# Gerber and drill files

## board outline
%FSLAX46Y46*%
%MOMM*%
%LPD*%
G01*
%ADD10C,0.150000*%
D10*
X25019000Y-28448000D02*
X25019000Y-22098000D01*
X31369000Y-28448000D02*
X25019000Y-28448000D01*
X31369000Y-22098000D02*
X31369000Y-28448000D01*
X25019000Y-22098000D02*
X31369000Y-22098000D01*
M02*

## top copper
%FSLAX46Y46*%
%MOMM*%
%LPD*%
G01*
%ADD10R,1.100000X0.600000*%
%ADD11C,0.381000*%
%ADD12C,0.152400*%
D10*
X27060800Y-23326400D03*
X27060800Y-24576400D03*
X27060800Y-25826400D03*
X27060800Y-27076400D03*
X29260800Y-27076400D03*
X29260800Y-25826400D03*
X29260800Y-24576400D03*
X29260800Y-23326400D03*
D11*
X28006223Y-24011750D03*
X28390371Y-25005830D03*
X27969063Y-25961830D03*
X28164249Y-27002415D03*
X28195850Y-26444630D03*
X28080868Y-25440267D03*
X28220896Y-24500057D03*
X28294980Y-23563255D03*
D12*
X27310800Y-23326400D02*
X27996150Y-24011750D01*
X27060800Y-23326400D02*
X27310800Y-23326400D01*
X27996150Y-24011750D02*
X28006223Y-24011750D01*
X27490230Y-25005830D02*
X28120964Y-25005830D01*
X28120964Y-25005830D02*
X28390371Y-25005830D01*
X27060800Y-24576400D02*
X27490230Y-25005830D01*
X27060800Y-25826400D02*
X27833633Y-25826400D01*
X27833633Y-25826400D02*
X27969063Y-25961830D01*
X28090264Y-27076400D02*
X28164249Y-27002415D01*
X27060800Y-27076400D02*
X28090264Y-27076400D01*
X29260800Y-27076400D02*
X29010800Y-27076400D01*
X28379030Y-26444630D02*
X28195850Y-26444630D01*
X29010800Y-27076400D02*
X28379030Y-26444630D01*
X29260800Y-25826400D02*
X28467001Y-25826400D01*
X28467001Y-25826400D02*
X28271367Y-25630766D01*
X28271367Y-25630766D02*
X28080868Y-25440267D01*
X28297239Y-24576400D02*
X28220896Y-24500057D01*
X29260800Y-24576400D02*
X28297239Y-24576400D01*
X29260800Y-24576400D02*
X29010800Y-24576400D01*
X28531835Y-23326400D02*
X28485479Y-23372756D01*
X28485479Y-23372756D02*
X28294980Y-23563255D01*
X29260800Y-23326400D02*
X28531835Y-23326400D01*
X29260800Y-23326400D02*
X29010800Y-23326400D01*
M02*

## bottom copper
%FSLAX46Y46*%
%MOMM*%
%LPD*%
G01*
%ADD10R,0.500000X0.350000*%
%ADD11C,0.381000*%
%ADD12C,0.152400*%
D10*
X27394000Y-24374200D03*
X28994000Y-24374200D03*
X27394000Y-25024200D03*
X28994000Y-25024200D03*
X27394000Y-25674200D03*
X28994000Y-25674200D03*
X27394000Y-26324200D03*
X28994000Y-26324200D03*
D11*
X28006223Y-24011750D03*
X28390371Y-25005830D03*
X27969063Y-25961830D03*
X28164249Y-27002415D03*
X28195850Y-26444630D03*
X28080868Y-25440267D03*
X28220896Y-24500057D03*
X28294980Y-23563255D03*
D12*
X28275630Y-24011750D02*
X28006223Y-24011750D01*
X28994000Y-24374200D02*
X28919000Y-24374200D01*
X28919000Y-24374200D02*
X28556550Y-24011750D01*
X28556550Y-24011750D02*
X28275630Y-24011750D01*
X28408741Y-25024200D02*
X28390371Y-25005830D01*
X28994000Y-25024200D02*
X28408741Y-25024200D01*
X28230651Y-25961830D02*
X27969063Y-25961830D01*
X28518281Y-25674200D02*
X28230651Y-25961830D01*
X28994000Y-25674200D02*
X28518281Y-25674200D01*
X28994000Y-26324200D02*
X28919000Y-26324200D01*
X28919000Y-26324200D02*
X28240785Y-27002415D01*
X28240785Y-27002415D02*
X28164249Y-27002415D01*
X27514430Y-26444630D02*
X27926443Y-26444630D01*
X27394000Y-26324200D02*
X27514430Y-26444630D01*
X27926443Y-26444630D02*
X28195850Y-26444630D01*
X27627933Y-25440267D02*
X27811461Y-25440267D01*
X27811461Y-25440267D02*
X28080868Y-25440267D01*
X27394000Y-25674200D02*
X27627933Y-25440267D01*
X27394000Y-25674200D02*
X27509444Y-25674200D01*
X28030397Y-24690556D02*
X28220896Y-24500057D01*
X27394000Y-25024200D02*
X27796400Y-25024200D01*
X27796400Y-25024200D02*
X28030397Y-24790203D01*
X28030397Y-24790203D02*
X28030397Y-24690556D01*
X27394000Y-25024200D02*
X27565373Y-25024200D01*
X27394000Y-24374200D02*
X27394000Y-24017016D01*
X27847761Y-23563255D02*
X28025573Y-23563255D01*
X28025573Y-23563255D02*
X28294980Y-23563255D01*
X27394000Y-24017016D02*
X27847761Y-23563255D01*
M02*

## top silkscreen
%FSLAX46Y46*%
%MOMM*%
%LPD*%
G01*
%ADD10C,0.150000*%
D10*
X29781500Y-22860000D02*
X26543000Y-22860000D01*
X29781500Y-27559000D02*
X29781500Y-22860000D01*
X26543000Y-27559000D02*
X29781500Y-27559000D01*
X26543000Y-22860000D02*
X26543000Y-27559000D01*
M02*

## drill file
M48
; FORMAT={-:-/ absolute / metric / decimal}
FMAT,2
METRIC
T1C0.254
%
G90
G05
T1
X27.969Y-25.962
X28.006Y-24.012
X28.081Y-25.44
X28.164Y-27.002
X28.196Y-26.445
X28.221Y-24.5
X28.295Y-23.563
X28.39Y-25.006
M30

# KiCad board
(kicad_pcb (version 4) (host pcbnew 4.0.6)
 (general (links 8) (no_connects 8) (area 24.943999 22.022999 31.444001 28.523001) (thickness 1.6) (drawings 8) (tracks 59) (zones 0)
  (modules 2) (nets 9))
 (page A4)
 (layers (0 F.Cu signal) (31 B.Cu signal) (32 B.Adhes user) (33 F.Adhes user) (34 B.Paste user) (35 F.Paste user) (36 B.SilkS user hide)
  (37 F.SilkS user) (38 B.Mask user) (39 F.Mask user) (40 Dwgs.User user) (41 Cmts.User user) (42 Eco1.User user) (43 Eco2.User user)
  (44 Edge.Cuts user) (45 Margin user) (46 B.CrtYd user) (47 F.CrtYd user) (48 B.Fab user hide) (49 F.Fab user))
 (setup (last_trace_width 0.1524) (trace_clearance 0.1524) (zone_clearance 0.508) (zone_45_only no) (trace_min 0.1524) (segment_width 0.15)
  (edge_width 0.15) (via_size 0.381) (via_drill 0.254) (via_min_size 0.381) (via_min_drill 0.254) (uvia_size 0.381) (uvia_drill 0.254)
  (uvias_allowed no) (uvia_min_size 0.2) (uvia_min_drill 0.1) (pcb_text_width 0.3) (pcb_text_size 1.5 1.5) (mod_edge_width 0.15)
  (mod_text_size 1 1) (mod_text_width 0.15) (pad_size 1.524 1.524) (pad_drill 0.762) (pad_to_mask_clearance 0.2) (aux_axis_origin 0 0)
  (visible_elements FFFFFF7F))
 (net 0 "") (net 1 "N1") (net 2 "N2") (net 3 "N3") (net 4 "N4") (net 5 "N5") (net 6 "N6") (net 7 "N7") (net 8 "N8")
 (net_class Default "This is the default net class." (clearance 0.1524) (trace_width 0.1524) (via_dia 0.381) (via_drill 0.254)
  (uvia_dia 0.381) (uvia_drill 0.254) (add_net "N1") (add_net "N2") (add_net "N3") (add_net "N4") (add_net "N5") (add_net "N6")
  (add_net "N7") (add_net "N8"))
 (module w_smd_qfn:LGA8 (layer F.Cu) (at 28.1608 25.2264)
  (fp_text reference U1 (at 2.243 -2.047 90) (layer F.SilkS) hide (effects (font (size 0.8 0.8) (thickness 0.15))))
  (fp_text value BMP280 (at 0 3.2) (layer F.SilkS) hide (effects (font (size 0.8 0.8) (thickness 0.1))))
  (pad 1 smd rect (at -1.1 -1.9) (size 1.1 0.6) (layers F.Cu F.Paste F.Mask) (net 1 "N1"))
  (pad 2 smd rect (at -1.1 -0.65) (size 1.1 0.6) (layers F.Cu F.Paste F.Mask) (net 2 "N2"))
  (pad 3 smd rect (at -1.1 0.6) (size 1.1 0.6) (layers F.Cu F.Paste F.Mask) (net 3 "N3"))
  (pad 4 smd rect (at -1.1 1.85) (size 1.1 0.6) (layers F.Cu F.Paste F.Mask) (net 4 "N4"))
  (pad 5 smd rect (at 1.1 1.85) (size 1.1 0.6) (layers F.Cu F.Paste F.Mask) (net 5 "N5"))
  (pad 6 smd rect (at 1.1 0.6) (size 1.1 0.6) (layers F.Cu F.Paste F.Mask) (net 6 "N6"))
  (pad 7 smd rect (at 1.1 -0.65) (size 1.1 0.6) (layers F.Cu F.Paste F.Mask) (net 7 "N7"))
  (pad 8 smd rect (at 1.1 -1.9) (size 1.1 0.6) (layers F.Cu F.Paste F.Mask) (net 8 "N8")))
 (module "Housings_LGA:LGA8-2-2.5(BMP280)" (layer B.Cu) (at 28.194 25.3492 270)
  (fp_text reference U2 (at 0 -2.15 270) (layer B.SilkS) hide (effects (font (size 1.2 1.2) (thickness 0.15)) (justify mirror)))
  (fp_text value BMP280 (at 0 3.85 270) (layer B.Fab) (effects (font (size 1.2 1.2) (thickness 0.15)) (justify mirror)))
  (pad 1 smd rect (at -0.975 0.8 270) (size 0.35 0.5) (layers B.Cu B.Paste B.Mask) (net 8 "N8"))
  (pad 8 smd rect (at -0.975 -0.8 270) (size 0.35 0.5) (layers B.Cu B.Paste B.Mask) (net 1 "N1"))
  (pad 2 smd rect (at -0.325 0.8 270) (size 0.35 0.5) (layers B.Cu B.Paste B.Mask) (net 7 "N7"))
  (pad 7 smd rect (at -0.325 -0.8 270) (size 0.35 0.5) (layers B.Cu B.Paste B.Mask) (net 2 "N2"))
  (pad 3 smd rect (at 0.325 0.8 270) (size 0.35 0.5) (layers B.Cu B.Paste B.Mask) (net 6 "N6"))
  (pad 6 smd rect (at 0.325 -0.8 270) (size 0.35 0.5) (layers B.Cu B.Paste B.Mask) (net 3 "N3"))
  (pad 4 smd rect (at 0.975 0.8 270) (size 0.35 0.5) (layers B.Cu B.Paste B.Mask) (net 5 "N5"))
  (pad 5 smd rect (at 0.975 -0.8 270) (size 0.35 0.5) (layers B.Cu B.Paste B.Mask) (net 4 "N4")))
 (gr_line (start 25.019 28.448) (end 25.019 22.098) (layer Edge.Cuts) (width 0.15))
 (gr_line (start 31.369 28.448) (end 25.019 28.448) (layer Edge.Cuts) (width 0.15))
 (gr_line (start 31.369 22.098) (end 31.369 28.448) (layer Edge.Cuts) (width 0.15))
 (gr_line (start 25.019 22.098) (end 31.369 22.098) (layer Edge.Cuts) (width 0.15))
 (gr_line (start 29.7815 22.86) (end 26.543 22.86) (layer F.SilkS) (width 0.15))
 (gr_line (start 29.7815 27.559) (end 29.7815 22.86) (layer F.SilkS) (width 0.15))
 (gr_line (start 26.543 27.559) (end 29.7815 27.559) (layer F.SilkS) (width 0.15))
 (gr_line (start 26.543 22.86) (end 26.543 27.559) (layer F.SilkS) (width 0.15))
 (segment (start 27.3108 23.3264) (end 27.99615 24.01175) (width 0.1524) (layer F.Cu) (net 1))
 (segment (start 28.27563 24.01175) (end 28.006223 24.01175) (width 0.1524) (layer B.Cu) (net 1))
 (segment (start 27.0608 23.3264) (end 27.3108 23.3264) (width 0.1524) (layer F.Cu) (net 1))
 (segment (start 28.994 24.3742) (end 28.919 24.3742) (width 0.1524) (layer B.Cu) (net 1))
 (segment (start 28.919 24.3742) (end 28.55655 24.01175) (width 0.1524) (layer B.Cu) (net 1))
 (segment (start 28.55655 24.01175) (end 28.27563 24.01175) (width 0.1524) (layer B.Cu) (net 1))
 (segment (start 27.99615 24.01175) (end 28.006223 24.01175) (width 0.1524) (layer F.Cu) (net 1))
 (via (at 28.006223 24.01175) (size 0.381) (drill 0.254) (layers F.Cu B.Cu) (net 1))
 (segment (start 28.408741 25.0242) (end 28.390371 25.00583) (width 0.1524) (layer B.Cu) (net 2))
 (segment (start 28.994 25.0242) (end 28.408741 25.0242) (width 0.1524) (layer B.Cu) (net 2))
 (segment (start 27.49023 25.00583) (end 28.120964 25.00583) (width 0.1524) (layer F.Cu) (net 2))
 (segment (start 28.120964 25.00583) (end 28.390371 25.00583) (width 0.1524) (layer F.Cu) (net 2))
 (segment (start 27.0608 24.5764) (end 27.49023 25.00583) (width 0.1524) (layer F.Cu) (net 2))
 (via (at 28.390371 25.00583) (size 0.381) (drill 0.254) (layers F.Cu B.Cu) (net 2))
 (segment (start 27.0608 25.8264) (end 27.833633 25.8264) (width 0.1524) (layer F.Cu) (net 3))
 (segment (start 28.230651 25.96183) (end 27.969063 25.96183) (width 0.1524) (layer B.Cu) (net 3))
 (segment (start 28.518281 25.6742) (end 28.230651 25.96183) (width 0.1524) (layer B.Cu) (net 3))
 (segment (start 28.994 25.6742) (end 28.518281 25.6742) (width 0.1524) (layer B.Cu) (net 3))
 (via (at 27.969063 25.96183) (size 0.381) (drill 0.254) (layers F.Cu B.Cu) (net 3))
 (segment (start 27.833633 25.8264) (end 27.969063 25.96183) (width 0.1524) (layer F.Cu) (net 3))
 (segment (start 28.090264 27.0764) (end 28.164249 27.002415) (width 0.1524) (layer F.Cu) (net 4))
 (segment (start 27.0608 27.0764) (end 28.090264 27.0764) (width 0.1524) (layer F.Cu) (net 4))
 (segment (start 28.994 26.3242) (end 28.919 26.3242) (width 0.1524) (layer B.Cu) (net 4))
 (segment (start 28.919 26.3242) (end 28.240785 27.002415) (width 0.1524) (layer B.Cu) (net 4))
 (segment (start 28.240785 27.002415) (end 28.164249 27.002415) (width 0.1524) (layer B.Cu) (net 4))
 (via (at 28.164249 27.002415) (size 0.381) (drill 0.254) (layers F.Cu B.Cu) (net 4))
 (segment (start 29.2608 27.0764) (end 29.0108 27.0764) (width 0.1524) (layer F.Cu) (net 5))
 (segment (start 27.51443 26.44463) (end 27.926443 26.44463) (width 0.1524) (layer B.Cu) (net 5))
 (segment (start 27.394 26.3242) (end 27.51443 26.44463) (width 0.1524) (layer B.Cu) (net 5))
 (segment (start 28.37903 26.44463) (end 28.19585 26.44463) (width 0.1524) (layer F.Cu) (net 5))
 (segment (start 29.0108 27.0764) (end 28.37903 26.44463) (width 0.1524) (layer F.Cu) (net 5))
 (via (at 28.19585 26.44463) (size 0.381) (drill 0.254) (layers F.Cu B.Cu) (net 5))
 (segment (start 27.926443 26.44463) (end 28.19585 26.44463) (width 0.1524) (layer B.Cu) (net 5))
 (segment (start 29.2608 25.8264) (end 28.467001 25.8264) (width 0.1524) (layer F.Cu) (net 6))
 (segment (start 27.627933 25.440267) (end 27.811461 25.440267) (width 0.1524) (layer B.Cu) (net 6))
 (segment (start 27.811461 25.440267) (end 28.080868 25.440267) (width 0.1524) (layer B.Cu) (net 6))
 (segment (start 28.467001 25.8264) (end 28.271367 25.630766) (width 0.1524) (layer F.Cu) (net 6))
 (segment (start 28.271367 25.630766) (end 28.080868 25.440267) (width 0.1524) (layer F.Cu) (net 6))
 (segment (start 27.394 25.6742) (end 27.627933 25.440267) (width 0.1524) (layer B.Cu) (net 6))
 (via (at 28.080868 25.440267) (size 0.381) (drill 0.254) (layers F.Cu B.Cu) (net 6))
 (segment (start 27.394 25.6742) (end 27.509444 25.6742) (width 0.1524) (layer B.Cu) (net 6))
 (segment (start 28.030397 24.690556) (end 28.220896 24.500057) (width 0.1524) (layer B.Cu) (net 7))
 (segment (start 27.394 25.0242) (end 27.7964 25.0242) (width 0.1524) (layer B.Cu) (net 7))
 (segment (start 28.297239 24.5764) (end 28.220896 24.500057) (width 0.1524) (layer F.Cu) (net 7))
 (segment (start 27.7964 25.0242) (end 28.030397 24.790203) (width 0.1524) (layer B.Cu) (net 7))
 (segment (start 28.030397 24.790203) (end 28.030397 24.690556) (width 0.1524) (layer B.Cu) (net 7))
 (segment (start 29.2608 24.5764) (end 28.297239 24.5764) (width 0.1524) (layer F.Cu) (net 7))
 (via (at 28.220896 24.500057) (size 0.381) (drill 0.254) (layers F.Cu B.Cu) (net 7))
 (segment (start 27.394 25.0242) (end 27.565373 25.0242) (width 0.1524) (layer B.Cu) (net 7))
 (segment (start 29.2608 24.5764) (end 29.0108 24.5764) (width 0.1524) (layer F.Cu) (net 7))
 (segment (start 28.531835 23.3264) (end 28.485479 23.372756) (width 0.1524) (layer F.Cu) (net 8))
 (segment (start 27.394 24.3742) (end 27.394 24.017016) (width 0.1524) (layer B.Cu) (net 8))
 (segment (start 27.847761 23.563255) (end 28.025573 23.563255) (width 0.1524) (layer B.Cu) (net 8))
 (segment (start 28.485479 23.372756) (end 28.29498 23.563255) (width 0.1524) (layer F.Cu) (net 8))
 (segment (start 28.025573 23.563255) (end 28.29498 23.563255) (width 0.1524) (layer B.Cu) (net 8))
 (segment (start 29.2608 23.3264) (end 28.531835 23.3264) (width 0.1524) (layer F.Cu) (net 8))
 (segment (start 27.394 24.017016) (end 27.847761 23.563255) (width 0.1524) (layer B.Cu) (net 8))
 (via (at 28.29498 23.563255) (size 0.381) (drill 0.254) (layers F.Cu B.Cu) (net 8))
 (segment (start 29.2608 23.3264) (end 29.0108 23.3264) (width 0.1524) (layer F.Cu) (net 8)))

